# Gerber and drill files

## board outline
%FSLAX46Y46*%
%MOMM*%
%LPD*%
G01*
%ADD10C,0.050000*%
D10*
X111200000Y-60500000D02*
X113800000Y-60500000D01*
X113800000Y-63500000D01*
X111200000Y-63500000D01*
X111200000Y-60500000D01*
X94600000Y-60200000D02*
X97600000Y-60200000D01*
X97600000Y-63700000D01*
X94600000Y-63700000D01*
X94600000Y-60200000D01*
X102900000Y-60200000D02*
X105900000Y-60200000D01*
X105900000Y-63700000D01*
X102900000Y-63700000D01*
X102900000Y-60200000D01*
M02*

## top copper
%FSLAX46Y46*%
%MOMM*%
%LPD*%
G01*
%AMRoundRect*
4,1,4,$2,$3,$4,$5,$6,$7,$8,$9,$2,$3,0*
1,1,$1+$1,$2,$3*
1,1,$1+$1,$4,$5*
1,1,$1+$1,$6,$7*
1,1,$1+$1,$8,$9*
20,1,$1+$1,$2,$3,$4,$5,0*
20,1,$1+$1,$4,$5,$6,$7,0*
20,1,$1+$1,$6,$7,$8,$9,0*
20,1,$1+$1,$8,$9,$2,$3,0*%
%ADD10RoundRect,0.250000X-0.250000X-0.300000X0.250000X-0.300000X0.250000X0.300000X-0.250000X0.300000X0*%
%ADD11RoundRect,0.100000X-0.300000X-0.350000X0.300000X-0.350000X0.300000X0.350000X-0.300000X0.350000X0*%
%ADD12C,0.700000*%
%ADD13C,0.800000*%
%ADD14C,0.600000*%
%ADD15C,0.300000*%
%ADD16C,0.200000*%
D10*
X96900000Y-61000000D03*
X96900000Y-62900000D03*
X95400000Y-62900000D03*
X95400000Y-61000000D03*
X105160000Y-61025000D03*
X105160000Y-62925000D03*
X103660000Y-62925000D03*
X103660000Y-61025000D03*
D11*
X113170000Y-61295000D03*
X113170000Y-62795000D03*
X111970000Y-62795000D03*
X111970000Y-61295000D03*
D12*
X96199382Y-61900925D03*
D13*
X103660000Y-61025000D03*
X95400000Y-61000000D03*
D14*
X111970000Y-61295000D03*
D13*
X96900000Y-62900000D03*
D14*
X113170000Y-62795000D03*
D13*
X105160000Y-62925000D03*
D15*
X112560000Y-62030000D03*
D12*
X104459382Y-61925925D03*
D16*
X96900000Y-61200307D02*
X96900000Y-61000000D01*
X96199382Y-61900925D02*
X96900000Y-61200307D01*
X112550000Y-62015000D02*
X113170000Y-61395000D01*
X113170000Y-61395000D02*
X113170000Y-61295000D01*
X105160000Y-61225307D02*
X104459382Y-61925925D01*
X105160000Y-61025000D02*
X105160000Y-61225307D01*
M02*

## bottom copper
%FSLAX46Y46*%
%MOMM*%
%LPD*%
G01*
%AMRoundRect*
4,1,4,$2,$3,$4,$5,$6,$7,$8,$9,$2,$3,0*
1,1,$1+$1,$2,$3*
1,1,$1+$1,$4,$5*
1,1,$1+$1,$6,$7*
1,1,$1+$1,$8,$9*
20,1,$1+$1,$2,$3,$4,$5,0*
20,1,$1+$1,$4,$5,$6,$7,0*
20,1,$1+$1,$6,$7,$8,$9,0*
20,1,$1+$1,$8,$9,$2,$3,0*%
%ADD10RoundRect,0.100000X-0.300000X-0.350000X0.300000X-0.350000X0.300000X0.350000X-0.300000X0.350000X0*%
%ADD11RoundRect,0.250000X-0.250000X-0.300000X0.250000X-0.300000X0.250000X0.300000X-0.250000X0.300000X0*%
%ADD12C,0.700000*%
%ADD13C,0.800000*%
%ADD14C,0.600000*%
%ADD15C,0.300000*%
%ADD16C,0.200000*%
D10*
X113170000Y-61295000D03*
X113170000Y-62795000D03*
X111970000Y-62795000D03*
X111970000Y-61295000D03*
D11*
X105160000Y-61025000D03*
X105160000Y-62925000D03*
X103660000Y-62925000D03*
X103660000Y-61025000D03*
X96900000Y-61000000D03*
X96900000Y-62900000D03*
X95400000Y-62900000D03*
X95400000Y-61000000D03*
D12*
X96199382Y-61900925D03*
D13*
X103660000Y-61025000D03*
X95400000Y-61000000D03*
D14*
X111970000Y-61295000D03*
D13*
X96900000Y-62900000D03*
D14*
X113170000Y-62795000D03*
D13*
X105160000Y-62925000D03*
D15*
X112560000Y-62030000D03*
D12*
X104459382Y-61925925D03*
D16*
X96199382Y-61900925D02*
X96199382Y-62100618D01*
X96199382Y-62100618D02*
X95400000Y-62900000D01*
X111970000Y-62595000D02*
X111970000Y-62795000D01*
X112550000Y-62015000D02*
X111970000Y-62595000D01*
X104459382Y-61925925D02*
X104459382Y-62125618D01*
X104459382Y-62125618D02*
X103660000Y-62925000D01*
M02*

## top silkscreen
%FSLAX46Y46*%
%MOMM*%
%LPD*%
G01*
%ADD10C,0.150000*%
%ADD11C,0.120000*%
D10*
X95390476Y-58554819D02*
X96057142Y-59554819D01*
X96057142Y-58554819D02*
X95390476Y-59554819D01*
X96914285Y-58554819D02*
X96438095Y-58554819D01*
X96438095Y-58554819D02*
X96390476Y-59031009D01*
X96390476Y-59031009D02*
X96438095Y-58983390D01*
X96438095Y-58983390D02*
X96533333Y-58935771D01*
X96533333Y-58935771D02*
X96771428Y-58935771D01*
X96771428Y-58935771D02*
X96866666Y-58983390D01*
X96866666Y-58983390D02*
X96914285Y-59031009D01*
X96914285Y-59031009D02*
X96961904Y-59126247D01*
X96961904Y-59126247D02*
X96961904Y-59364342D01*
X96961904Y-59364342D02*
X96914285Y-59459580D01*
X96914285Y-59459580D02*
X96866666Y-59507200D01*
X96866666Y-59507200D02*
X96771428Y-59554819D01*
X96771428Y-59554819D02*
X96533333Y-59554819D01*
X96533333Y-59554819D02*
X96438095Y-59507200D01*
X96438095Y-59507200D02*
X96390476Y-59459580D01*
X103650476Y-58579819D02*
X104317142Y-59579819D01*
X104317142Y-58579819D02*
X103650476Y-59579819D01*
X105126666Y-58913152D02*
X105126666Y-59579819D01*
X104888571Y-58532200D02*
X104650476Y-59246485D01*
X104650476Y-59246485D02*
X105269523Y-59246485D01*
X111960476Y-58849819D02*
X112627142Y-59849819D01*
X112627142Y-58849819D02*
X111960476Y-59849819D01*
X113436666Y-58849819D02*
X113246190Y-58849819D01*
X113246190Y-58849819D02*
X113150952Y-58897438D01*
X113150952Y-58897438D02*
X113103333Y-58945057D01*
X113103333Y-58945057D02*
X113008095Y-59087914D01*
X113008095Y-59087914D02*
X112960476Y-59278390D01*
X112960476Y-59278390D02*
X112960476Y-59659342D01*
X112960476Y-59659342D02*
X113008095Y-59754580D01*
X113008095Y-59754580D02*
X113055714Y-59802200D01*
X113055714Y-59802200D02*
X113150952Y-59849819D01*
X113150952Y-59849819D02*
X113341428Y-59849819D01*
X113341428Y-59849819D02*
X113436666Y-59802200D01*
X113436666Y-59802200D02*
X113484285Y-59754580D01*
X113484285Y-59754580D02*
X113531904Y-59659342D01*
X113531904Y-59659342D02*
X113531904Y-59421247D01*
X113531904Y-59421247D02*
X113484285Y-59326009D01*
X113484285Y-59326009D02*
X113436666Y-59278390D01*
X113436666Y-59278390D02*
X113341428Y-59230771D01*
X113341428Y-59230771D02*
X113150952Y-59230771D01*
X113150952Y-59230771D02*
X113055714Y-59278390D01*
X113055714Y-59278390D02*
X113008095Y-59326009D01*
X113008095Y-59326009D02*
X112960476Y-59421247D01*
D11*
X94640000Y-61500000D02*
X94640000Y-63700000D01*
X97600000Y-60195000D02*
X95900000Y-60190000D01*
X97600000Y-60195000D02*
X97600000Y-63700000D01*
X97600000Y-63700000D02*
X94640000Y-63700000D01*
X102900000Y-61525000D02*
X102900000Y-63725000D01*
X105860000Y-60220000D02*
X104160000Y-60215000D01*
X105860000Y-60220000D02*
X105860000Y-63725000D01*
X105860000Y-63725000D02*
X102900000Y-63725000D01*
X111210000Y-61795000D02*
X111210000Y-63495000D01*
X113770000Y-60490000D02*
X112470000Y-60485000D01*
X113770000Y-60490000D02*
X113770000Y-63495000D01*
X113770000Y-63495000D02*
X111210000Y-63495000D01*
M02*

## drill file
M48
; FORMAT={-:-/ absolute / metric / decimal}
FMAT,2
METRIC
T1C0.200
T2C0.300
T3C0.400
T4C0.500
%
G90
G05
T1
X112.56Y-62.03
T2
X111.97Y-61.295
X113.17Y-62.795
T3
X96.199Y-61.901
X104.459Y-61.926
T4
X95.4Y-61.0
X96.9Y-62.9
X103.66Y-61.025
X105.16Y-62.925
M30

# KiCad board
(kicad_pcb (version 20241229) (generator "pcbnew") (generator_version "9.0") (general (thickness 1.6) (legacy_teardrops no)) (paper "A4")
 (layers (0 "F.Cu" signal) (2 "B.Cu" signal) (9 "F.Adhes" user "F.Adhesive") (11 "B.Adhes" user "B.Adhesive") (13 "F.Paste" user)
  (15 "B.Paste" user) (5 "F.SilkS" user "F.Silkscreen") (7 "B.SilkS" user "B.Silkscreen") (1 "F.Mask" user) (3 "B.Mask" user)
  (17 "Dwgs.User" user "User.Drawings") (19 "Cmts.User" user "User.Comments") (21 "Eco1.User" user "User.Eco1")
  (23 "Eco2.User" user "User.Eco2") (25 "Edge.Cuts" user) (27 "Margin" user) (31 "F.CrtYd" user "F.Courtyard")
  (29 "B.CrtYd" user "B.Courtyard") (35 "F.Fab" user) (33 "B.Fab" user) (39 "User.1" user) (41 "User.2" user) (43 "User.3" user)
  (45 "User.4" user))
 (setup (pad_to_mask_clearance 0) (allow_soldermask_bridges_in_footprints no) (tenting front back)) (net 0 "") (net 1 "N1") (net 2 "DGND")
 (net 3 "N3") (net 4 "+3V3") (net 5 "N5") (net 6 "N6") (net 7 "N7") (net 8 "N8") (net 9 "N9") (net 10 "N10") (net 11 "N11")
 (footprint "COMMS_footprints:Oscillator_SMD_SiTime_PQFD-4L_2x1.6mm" (layer "F.Cu") (at 112.77 62.395)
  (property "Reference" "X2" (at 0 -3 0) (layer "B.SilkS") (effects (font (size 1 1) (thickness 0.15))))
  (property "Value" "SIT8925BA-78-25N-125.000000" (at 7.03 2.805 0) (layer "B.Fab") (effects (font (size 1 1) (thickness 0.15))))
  (pad "1" smd roundrect (at 0.4 -1.1) (size 0.8 0.9) (layers "F.Mask" "B.Cu" "F.Paste") (roundrect_rratio 0.125) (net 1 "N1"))
  (pad "2" smd roundrect (at 0.4 0.4) (size 0.8 0.9) (layers "F.Mask" "B.Cu" "F.Paste") (roundrect_rratio 0.125) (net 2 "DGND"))
  (pad "3" smd roundrect (at -0.8 0.4) (size 0.8 0.9) (layers "F.Mask" "B.Cu" "F.Paste") (roundrect_rratio 0.125) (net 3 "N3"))
  (pad "4" smd roundrect (at -0.8 -1.1) (size 0.8 0.9) (layers "F.Mask" "B.Cu" "F.Paste") (roundrect_rratio 0.125) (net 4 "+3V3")))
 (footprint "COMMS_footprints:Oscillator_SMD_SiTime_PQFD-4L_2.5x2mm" (layer "F.Cu") (at 96.2 62.1)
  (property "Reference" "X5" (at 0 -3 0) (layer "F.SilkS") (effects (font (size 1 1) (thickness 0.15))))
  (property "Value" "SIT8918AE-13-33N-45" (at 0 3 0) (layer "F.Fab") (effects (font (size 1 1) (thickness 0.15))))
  (fp_line (start -1.56 -0.6) (end -1.56 1.6) (stroke (width 0.12) (type solid)) (layer "F.SilkS"))
  (fp_line (start 1.4 -1.905) (end -0.3 -1.91) (stroke (width 0.12) (type solid)) (layer "F.SilkS"))
  (fp_line (start 1.4 -1.905) (end 1.4 1.6) (stroke (width 0.12) (type solid)) (layer "F.SilkS"))
  (fp_line (start 1.4 1.6) (end -1.56 1.6) (stroke (width 0.12) (type solid)) (layer "F.SilkS"))
  (pad "1" smd roundrect (at 0.7 -1.1) (size 1 1.1) (layers "F.Cu" "F.Mask" "F.Paste") (roundrect_rratio 0.25) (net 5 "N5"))
  (pad "2" smd roundrect (at 0.7 0.8) (size 1 1.1) (layers "F.Cu" "F.Mask" "F.Paste") (roundrect_rratio 0.25) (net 2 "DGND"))
  (pad "3" smd roundrect (at -0.8 0.8) (size 1 1.1) (layers "F.Cu" "F.Mask" "F.Paste") (roundrect_rratio 0.25) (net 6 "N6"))
  (pad "4" smd roundrect (at -0.8 -1.1) (size 1 1.1) (layers "F.Cu" "F.Mask" "F.Paste") (roundrect_rratio 0.25) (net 4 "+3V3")))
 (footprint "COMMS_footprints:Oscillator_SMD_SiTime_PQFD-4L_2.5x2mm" (layer "F.Cu") (at 104.46 62.125)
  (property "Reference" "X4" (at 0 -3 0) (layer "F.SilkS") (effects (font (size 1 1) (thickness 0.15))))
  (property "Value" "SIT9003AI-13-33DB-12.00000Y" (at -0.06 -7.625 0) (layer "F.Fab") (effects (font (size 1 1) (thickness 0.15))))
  (fp_line (start -1.56 -0.6) (end -1.56 1.6) (stroke (width 0.12) (type solid)) (layer "F.SilkS"))
  (fp_line (start 1.4 -1.905) (end -0.3 -1.91) (stroke (width 0.12) (type solid)) (layer "F.SilkS"))
  (fp_line (start 1.4 -1.905) (end 1.4 1.6) (stroke (width 0.12) (type solid)) (layer "F.SilkS"))
  (fp_line (start 1.4 1.6) (end -1.56 1.6) (stroke (width 0.12) (type solid)) (layer "F.SilkS"))
  (pad "1" smd roundrect (at 0.7 -1.1) (size 1 1.1) (layers "F.Cu" "F.Mask" "F.Paste") (roundrect_rratio 0.25) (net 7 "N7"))
  (pad "2" smd roundrect (at 0.7 0.8) (size 1 1.1) (layers "F.Cu" "F.Mask" "F.Paste") (roundrect_rratio 0.25) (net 2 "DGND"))
  (pad "3" smd roundrect (at -0.8 0.8) (size 1 1.1) (layers "F.Cu" "F.Mask" "F.Paste") (roundrect_rratio 0.25) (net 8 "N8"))
  (pad "4" smd roundrect (at -0.8 -1.1) (size 1 1.1) (layers "F.Cu" "F.Mask" "F.Paste") (roundrect_rratio 0.25) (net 4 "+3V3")))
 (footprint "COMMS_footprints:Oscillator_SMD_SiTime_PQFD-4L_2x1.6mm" (layer "F.Cu") (at 112.77 62.395)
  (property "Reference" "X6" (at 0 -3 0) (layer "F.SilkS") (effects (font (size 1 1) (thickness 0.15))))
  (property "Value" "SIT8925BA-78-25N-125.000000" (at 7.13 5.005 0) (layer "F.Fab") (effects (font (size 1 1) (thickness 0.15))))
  (fp_line (start -1.56 -0.6) (end -1.56 1.1) (stroke (width 0.12) (type solid)) (layer "F.SilkS"))
  (fp_line (start 1 -1.905) (end -0.3 -1.91) (stroke (width 0.12) (type solid)) (layer "F.SilkS"))
  (fp_line (start 1 -1.905) (end 1 1.1) (stroke (width 0.12) (type solid)) (layer "F.SilkS"))
  (fp_line (start 1 1.1) (end -1.56 1.1) (stroke (width 0.12) (type solid)) (layer "F.SilkS"))
  (pad "1" smd roundrect (at 0.4 -1.1) (size 0.8 0.9) (layers "F.Cu" "F.Mask" "F.Paste") (roundrect_rratio 0.125) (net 3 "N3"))
  (pad "2" smd roundrect (at 0.4 0.4) (size 0.8 0.9) (layers "F.Cu" "F.Mask" "F.Paste") (roundrect_rratio 0.125) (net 2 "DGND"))
  (pad "3" smd roundrect (at -0.8 0.4) (size 0.8 0.9) (layers "F.Cu" "F.Mask" "F.Paste") (roundrect_rratio 0.125) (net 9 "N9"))
  (pad "4" smd roundrect (at -0.8 -1.1) (size 0.8 0.9) (layers "F.Cu" "F.Mask" "F.Paste") (roundrect_rratio 0.125) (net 4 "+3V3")))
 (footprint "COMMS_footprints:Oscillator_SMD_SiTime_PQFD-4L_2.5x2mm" (layer "F.Cu") (at 104.46 62.125)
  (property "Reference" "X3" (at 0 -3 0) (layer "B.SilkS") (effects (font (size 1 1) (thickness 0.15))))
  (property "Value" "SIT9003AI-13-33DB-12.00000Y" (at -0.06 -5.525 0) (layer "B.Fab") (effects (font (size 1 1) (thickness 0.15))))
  (pad "1" smd roundrect (at 0.7 -1.1) (size 1 1.1) (layers "F.Mask" "B.Cu" "F.Paste") (roundrect_rratio 0.25) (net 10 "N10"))
  (pad "2" smd roundrect (at 0.7 0.8) (size 1 1.1) (layers "F.Mask" "B.Cu" "F.Paste") (roundrect_rratio 0.25) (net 2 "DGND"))
  (pad "3" smd roundrect (at -0.8 0.8) (size 1 1.1) (layers "F.Mask" "B.Cu" "F.Paste") (roundrect_rratio 0.25) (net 7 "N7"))
  (pad "4" smd roundrect (at -0.8 -1.1) (size 1 1.1) (layers "F.Mask" "B.Cu" "F.Paste") (roundrect_rratio 0.25) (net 4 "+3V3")))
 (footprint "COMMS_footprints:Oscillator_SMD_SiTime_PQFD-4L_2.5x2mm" (layer "F.Cu") (at 96.2 62.1)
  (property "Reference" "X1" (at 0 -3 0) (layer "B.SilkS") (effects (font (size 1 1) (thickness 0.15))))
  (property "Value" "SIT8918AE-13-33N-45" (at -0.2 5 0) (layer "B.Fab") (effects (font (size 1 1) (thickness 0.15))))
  (pad "1" smd roundrect (at 0.7 -1.1) (size 1 1.1) (layers "F.Mask" "B.Cu" "F.Paste") (roundrect_rratio 0.25) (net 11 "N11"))
  (pad "2" smd roundrect (at 0.7 0.8) (size 1 1.1) (layers "F.Mask" "B.Cu" "F.Paste") (roundrect_rratio 0.25) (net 2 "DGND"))
  (pad "3" smd roundrect (at -0.8 0.8) (size 1 1.1) (layers "F.Mask" "B.Cu" "F.Paste") (roundrect_rratio 0.25) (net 5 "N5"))
  (pad "4" smd roundrect (at -0.8 -1.1) (size 1 1.1) (layers "F.Mask" "B.Cu" "F.Paste") (roundrect_rratio 0.25) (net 4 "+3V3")))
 (gr_rect (start 111.2 60.5) (end 113.8 63.5) (stroke (width 0.05) (type default)) (fill no) (layer "Edge.Cuts"))
 (gr_rect (start 94.6 60.2) (end 97.6 63.7) (stroke (width 0.05) (type default)) (fill no) (layer "Edge.Cuts"))
 (gr_rect (start 102.9 60.2) (end 105.9 63.7) (stroke (width 0.05) (type default)) (fill no) (layer "Edge.Cuts"))
 (segment (start 96.9 61.200307) (end 96.9 61) (width 0.2) (layer "F.Cu") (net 5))
 (segment (start 96.199382 61.900925) (end 96.9 61.200307) (width 0.2) (layer "F.Cu") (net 5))
 (via (at 96.199382 61.900925) (size 0.7) (drill 0.4) (layers "F.Cu" "B.Cu") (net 5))
 (segment (start 96.199382 61.900925) (end 96.199382 62.100618) (width 0.2) (layer "B.Cu") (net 5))
 (segment (start 96.199382 62.100618) (end 95.4 62.9) (width 0.2) (layer "B.Cu") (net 5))
 (via (at 103.66 61.025) (size 0.8) (drill 0.5) (layers "F.Cu" "B.Cu") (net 4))
 (via (at 95.4 61) (size 0.8) (drill 0.5) (layers "F.Cu" "B.Cu") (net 4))
 (via (at 111.97 61.295) (size 0.6) (drill 0.3) (layers "F.Cu" "B.Cu") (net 4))
 (via (at 96.9 62.9) (size 0.8) (drill 0.5) (layers "F.Cu" "B.Cu") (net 2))
 (via (at 113.17 62.795) (size 0.6) (drill 0.3) (layers "F.Cu" "B.Cu") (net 2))
 (via (at 105.16 62.925) (size 0.8) (drill 0.5) (layers "F.Cu" "B.Cu") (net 2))
 (segment (start 112.55 62.015) (end 113.17 61.395) (width 0.2) (layer "F.Cu") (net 3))
 (segment (start 113.17 61.395) (end 113.17 61.295) (width 0.2) (layer "F.Cu") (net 3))
 (via (at 112.56 62.03) (size 0.3) (drill 0.2) (layers "F.Cu" "B.Cu") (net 3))
 (segment (start 111.97 62.595) (end 111.97 62.795) (width 0.2) (layer "B.Cu") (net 3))
 (segment (start 112.55 62.015) (end 111.97 62.595) (width 0.2) (layer "B.Cu") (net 3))
 (segment (start 105.16 61.225307) (end 104.459382 61.925925) (width 0.2) (layer "F.Cu") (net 7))
 (segment (start 105.16 61.025) (end 105.16 61.225307) (width 0.2) (layer "F.Cu") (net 7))
 (via (at 104.459382 61.925925) (size 0.7) (drill 0.4) (layers "F.Cu" "B.Cu") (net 7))
 (segment (start 104.459382 61.925925) (end 104.459382 62.125618) (width 0.2) (layer "B.Cu") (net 7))
 (segment (start 104.459382 62.125618) (end 103.66 62.925) (width 0.2) (layer "B.Cu") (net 7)))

